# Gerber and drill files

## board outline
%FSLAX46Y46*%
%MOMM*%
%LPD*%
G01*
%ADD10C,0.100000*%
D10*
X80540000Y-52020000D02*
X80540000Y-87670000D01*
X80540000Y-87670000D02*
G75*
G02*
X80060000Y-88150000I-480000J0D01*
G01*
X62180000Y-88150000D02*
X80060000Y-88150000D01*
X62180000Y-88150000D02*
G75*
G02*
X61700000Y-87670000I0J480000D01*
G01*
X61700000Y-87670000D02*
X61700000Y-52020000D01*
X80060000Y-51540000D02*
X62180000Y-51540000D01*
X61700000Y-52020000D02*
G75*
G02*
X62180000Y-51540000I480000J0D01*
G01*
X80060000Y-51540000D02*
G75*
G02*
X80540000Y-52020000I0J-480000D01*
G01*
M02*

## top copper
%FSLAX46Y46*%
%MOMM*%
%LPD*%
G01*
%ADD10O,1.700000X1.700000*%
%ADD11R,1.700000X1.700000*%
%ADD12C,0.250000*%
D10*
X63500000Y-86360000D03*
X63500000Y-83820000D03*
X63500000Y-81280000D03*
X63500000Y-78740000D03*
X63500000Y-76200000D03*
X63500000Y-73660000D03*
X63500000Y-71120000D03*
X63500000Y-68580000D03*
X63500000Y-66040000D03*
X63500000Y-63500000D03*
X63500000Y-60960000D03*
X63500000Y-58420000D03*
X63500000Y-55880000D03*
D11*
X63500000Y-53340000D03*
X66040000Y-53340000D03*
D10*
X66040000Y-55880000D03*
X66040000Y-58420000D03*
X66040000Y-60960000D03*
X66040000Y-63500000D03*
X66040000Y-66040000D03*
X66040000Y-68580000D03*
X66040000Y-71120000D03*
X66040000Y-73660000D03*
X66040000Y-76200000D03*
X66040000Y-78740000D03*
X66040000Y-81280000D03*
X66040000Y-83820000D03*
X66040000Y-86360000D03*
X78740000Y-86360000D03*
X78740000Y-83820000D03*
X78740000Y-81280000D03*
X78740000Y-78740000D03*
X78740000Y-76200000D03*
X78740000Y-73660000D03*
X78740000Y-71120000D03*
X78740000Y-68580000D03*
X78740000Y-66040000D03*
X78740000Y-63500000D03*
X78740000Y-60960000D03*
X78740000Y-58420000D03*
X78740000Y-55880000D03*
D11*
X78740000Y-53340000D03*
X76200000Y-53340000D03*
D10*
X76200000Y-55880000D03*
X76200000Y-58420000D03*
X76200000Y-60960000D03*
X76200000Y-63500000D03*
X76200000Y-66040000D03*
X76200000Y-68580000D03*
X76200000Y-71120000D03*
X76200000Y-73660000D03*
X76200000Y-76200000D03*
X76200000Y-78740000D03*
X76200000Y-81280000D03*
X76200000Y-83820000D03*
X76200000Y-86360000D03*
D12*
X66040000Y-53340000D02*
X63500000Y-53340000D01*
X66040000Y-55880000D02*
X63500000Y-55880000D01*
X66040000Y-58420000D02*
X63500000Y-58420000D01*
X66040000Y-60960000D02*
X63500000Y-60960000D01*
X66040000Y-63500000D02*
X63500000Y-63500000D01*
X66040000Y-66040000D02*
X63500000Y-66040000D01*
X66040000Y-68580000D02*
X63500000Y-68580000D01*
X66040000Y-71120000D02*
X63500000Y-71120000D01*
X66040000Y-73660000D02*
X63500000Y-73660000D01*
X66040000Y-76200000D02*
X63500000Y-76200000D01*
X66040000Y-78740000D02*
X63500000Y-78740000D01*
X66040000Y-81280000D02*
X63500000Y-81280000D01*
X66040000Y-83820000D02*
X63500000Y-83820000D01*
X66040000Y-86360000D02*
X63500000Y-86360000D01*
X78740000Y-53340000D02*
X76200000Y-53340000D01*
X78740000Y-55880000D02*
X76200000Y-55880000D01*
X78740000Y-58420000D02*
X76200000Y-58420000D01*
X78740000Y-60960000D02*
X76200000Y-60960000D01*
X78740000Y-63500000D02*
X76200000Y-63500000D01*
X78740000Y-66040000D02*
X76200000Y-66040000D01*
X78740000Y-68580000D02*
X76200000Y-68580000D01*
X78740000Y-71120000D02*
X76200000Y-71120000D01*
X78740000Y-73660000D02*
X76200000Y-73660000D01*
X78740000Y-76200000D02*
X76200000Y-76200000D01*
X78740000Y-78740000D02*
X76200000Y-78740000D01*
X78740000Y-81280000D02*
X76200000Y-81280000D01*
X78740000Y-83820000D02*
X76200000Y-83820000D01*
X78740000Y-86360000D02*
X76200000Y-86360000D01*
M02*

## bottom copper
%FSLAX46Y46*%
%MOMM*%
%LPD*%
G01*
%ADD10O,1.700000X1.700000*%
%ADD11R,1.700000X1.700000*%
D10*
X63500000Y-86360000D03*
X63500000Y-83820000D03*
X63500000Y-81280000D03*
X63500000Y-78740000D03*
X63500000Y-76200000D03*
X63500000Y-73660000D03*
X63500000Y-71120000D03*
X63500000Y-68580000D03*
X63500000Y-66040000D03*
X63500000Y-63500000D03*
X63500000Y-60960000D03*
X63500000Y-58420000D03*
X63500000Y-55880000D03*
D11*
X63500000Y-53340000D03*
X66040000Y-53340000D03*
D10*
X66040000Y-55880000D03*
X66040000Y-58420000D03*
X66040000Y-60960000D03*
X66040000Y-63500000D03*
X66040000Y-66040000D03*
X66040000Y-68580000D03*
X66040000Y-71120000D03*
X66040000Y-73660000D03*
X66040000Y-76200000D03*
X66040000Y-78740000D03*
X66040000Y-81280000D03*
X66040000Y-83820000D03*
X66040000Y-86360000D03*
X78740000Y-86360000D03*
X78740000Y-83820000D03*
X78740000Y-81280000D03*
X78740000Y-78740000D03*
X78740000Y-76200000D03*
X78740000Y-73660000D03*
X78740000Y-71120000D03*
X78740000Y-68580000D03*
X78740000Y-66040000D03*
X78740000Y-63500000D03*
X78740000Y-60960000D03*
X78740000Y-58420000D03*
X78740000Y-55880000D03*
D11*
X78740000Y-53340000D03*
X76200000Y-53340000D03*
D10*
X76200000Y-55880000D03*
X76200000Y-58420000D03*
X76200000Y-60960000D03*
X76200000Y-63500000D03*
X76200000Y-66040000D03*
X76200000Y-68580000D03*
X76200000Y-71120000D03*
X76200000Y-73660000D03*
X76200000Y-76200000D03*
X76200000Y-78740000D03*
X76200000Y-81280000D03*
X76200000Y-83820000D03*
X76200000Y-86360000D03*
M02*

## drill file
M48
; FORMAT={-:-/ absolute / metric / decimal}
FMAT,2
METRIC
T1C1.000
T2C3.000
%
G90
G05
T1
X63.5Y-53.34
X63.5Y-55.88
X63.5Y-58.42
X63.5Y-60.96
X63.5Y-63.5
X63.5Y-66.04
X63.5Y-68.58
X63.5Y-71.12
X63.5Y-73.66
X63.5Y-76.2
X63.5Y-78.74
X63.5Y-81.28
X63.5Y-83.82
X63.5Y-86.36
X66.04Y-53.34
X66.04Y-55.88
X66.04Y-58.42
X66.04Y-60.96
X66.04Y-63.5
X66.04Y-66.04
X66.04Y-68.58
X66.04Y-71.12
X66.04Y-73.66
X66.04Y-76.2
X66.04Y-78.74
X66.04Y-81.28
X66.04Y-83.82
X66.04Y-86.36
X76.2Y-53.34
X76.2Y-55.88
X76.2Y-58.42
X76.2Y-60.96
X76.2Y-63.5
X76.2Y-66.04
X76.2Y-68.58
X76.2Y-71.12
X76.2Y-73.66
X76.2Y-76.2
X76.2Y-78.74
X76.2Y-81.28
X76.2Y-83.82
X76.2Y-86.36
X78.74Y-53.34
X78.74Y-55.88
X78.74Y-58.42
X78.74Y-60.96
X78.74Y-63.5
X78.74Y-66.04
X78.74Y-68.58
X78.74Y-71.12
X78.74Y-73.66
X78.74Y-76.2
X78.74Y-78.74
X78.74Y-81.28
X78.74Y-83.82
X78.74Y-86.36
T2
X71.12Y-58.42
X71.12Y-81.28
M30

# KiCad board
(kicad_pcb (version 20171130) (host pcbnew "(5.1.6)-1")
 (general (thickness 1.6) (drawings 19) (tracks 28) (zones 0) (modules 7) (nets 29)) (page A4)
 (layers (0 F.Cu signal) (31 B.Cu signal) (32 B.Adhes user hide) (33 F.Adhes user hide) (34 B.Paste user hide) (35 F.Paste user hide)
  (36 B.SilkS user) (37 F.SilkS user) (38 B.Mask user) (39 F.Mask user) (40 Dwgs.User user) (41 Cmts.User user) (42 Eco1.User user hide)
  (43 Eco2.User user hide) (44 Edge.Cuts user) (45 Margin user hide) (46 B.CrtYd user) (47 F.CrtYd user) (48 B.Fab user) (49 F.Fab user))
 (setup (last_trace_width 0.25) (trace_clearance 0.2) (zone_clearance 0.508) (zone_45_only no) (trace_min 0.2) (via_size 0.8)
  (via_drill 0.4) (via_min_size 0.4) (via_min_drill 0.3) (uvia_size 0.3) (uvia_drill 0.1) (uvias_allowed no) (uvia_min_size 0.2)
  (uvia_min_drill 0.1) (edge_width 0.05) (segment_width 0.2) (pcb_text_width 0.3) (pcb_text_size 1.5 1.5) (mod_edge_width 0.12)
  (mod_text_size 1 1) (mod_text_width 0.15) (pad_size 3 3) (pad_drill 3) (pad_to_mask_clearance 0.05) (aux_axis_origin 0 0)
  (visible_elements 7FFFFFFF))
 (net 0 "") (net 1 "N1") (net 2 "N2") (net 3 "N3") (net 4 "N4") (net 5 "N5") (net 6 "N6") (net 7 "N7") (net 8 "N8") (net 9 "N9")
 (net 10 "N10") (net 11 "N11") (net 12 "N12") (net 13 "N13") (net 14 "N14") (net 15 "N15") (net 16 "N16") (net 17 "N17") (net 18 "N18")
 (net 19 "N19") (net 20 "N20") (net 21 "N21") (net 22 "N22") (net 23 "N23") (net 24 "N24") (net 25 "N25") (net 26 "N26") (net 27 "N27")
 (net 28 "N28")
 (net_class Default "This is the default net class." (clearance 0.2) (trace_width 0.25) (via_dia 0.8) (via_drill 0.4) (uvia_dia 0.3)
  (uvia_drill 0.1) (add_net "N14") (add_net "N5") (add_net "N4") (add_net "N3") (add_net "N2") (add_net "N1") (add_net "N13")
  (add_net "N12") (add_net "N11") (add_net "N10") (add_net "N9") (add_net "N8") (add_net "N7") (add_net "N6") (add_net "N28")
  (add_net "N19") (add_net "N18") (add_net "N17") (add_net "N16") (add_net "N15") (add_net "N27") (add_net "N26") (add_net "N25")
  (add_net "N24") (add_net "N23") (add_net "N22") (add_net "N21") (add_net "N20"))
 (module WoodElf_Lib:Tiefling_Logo (layer F.Cu) (at 71.12 66.04 270)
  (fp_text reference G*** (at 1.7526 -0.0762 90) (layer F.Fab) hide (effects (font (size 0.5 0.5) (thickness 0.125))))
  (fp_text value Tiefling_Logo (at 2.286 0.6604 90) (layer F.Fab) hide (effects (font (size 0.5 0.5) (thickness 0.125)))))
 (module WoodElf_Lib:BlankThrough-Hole (layer F.Cu) (at 71.12 81.28)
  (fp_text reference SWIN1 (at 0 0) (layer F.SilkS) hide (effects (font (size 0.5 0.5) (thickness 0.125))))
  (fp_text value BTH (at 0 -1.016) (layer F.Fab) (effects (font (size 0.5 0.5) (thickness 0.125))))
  (pad "" np_thru_hole circle (at 0 0) (size 3 3) (drill 3) (layers *.Cu *.Mask) (solder_mask_margin 0.1) (clearance 0.1)))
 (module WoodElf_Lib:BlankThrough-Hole (layer F.Cu) (at 71.12 58.42)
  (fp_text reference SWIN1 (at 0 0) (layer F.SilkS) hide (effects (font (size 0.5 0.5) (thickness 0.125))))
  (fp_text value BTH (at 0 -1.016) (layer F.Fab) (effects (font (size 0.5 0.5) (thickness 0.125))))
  (pad "" np_thru_hole circle (at 0 0) (size 3 3) (drill 3) (layers *.Cu *.Mask) (solder_mask_margin 0.1) (clearance 0.1)))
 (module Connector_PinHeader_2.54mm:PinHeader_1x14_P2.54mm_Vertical (layer B.Cu) (at 63.5 53.34 180)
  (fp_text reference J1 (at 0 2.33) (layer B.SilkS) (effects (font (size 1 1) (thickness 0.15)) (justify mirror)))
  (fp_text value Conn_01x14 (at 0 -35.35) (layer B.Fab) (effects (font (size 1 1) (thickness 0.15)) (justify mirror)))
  (pad 14 thru_hole oval (at 0 -33.02 180) (size 1.7 1.7) (drill 1) (layers *.Cu *.Mask) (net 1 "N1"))
  (pad 13 thru_hole oval (at 0 -30.48 180) (size 1.7 1.7) (drill 1) (layers *.Cu *.Mask) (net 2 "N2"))
  (pad 12 thru_hole oval (at 0 -27.94 180) (size 1.7 1.7) (drill 1) (layers *.Cu *.Mask) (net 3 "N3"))
  (pad 11 thru_hole oval (at 0 -25.4 180) (size 1.7 1.7) (drill 1) (layers *.Cu *.Mask) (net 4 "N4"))
  (pad 10 thru_hole oval (at 0 -22.86 180) (size 1.7 1.7) (drill 1) (layers *.Cu *.Mask) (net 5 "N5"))
  (pad 9 thru_hole oval (at 0 -20.32 180) (size 1.7 1.7) (drill 1) (layers *.Cu *.Mask) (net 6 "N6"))
  (pad 8 thru_hole oval (at 0 -17.78 180) (size 1.7 1.7) (drill 1) (layers *.Cu *.Mask) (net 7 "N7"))
  (pad 7 thru_hole oval (at 0 -15.24 180) (size 1.7 1.7) (drill 1) (layers *.Cu *.Mask) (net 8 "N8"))
  (pad 6 thru_hole oval (at 0 -12.7 180) (size 1.7 1.7) (drill 1) (layers *.Cu *.Mask) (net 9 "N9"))
  (pad 5 thru_hole oval (at 0 -10.16 180) (size 1.7 1.7) (drill 1) (layers *.Cu *.Mask) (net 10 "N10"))
  (pad 4 thru_hole oval (at 0 -7.62 180) (size 1.7 1.7) (drill 1) (layers *.Cu *.Mask) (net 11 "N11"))
  (pad 3 thru_hole oval (at 0 -5.08 180) (size 1.7 1.7) (drill 1) (layers *.Cu *.Mask) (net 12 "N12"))
  (pad 2 thru_hole oval (at 0 -2.54 180) (size 1.7 1.7) (drill 1) (layers *.Cu *.Mask) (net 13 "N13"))
  (pad 1 thru_hole rect (at 0 0 180) (size 1.7 1.7) (drill 1) (layers *.Cu *.Mask) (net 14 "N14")))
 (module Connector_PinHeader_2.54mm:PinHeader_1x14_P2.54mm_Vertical (layer F.Cu) (at 66.04 53.34)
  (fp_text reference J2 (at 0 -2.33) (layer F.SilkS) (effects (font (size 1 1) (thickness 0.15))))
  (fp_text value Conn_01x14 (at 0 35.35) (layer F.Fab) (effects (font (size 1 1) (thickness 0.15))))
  (pad 1 thru_hole rect (at 0 0) (size 1.7 1.7) (drill 1) (layers *.Cu *.Mask) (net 14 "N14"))
  (pad 2 thru_hole oval (at 0 2.54) (size 1.7 1.7) (drill 1) (layers *.Cu *.Mask) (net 13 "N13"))
  (pad 3 thru_hole oval (at 0 5.08) (size 1.7 1.7) (drill 1) (layers *.Cu *.Mask) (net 12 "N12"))
  (pad 4 thru_hole oval (at 0 7.62) (size 1.7 1.7) (drill 1) (layers *.Cu *.Mask) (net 11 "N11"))
  (pad 5 thru_hole oval (at 0 10.16) (size 1.7 1.7) (drill 1) (layers *.Cu *.Mask) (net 10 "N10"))
  (pad 6 thru_hole oval (at 0 12.7) (size 1.7 1.7) (drill 1) (layers *.Cu *.Mask) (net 9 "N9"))
  (pad 7 thru_hole oval (at 0 15.24) (size 1.7 1.7) (drill 1) (layers *.Cu *.Mask) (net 8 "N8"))
  (pad 8 thru_hole oval (at 0 17.78) (size 1.7 1.7) (drill 1) (layers *.Cu *.Mask) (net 7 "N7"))
  (pad 9 thru_hole oval (at 0 20.32) (size 1.7 1.7) (drill 1) (layers *.Cu *.Mask) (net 6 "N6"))
  (pad 10 thru_hole oval (at 0 22.86) (size 1.7 1.7) (drill 1) (layers *.Cu *.Mask) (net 5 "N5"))
  (pad 11 thru_hole oval (at 0 25.4) (size 1.7 1.7) (drill 1) (layers *.Cu *.Mask) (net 4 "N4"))
  (pad 12 thru_hole oval (at 0 27.94) (size 1.7 1.7) (drill 1) (layers *.Cu *.Mask) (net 3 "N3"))
  (pad 13 thru_hole oval (at 0 30.48) (size 1.7 1.7) (drill 1) (layers *.Cu *.Mask) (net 2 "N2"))
  (pad 14 thru_hole oval (at 0 33.02) (size 1.7 1.7) (drill 1) (layers *.Cu *.Mask) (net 1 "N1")))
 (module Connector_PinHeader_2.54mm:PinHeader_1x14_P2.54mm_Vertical (layer B.Cu) (at 78.74 53.34 180)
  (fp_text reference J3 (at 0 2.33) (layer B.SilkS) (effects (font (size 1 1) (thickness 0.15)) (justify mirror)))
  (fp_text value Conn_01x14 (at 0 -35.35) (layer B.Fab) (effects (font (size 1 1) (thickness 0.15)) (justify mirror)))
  (pad 14 thru_hole oval (at 0 -33.02 180) (size 1.7 1.7) (drill 1) (layers *.Cu *.Mask) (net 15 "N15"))
  (pad 13 thru_hole oval (at 0 -30.48 180) (size 1.7 1.7) (drill 1) (layers *.Cu *.Mask) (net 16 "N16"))
  (pad 12 thru_hole oval (at 0 -27.94 180) (size 1.7 1.7) (drill 1) (layers *.Cu *.Mask) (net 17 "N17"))
  (pad 11 thru_hole oval (at 0 -25.4 180) (size 1.7 1.7) (drill 1) (layers *.Cu *.Mask) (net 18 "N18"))
  (pad 10 thru_hole oval (at 0 -22.86 180) (size 1.7 1.7) (drill 1) (layers *.Cu *.Mask) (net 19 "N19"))
  (pad 9 thru_hole oval (at 0 -20.32 180) (size 1.7 1.7) (drill 1) (layers *.Cu *.Mask) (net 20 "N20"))
  (pad 8 thru_hole oval (at 0 -17.78 180) (size 1.7 1.7) (drill 1) (layers *.Cu *.Mask) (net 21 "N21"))
  (pad 7 thru_hole oval (at 0 -15.24 180) (size 1.7 1.7) (drill 1) (layers *.Cu *.Mask) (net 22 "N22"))
  (pad 6 thru_hole oval (at 0 -12.7 180) (size 1.7 1.7) (drill 1) (layers *.Cu *.Mask) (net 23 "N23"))
  (pad 5 thru_hole oval (at 0 -10.16 180) (size 1.7 1.7) (drill 1) (layers *.Cu *.Mask) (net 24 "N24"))
  (pad 4 thru_hole oval (at 0 -7.62 180) (size 1.7 1.7) (drill 1) (layers *.Cu *.Mask) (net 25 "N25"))
  (pad 3 thru_hole oval (at 0 -5.08 180) (size 1.7 1.7) (drill 1) (layers *.Cu *.Mask) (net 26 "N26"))
  (pad 2 thru_hole oval (at 0 -2.54 180) (size 1.7 1.7) (drill 1) (layers *.Cu *.Mask) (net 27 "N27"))
  (pad 1 thru_hole rect (at 0 0 180) (size 1.7 1.7) (drill 1) (layers *.Cu *.Mask) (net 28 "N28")))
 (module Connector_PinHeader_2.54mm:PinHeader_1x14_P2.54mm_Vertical (layer F.Cu) (at 76.2 53.34)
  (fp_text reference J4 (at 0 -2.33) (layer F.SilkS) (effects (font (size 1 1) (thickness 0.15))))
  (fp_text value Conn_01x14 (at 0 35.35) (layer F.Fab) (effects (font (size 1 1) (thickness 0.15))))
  (pad 1 thru_hole rect (at 0 0) (size 1.7 1.7) (drill 1) (layers *.Cu *.Mask) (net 28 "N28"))
  (pad 2 thru_hole oval (at 0 2.54) (size 1.7 1.7) (drill 1) (layers *.Cu *.Mask) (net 27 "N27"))
  (pad 3 thru_hole oval (at 0 5.08) (size 1.7 1.7) (drill 1) (layers *.Cu *.Mask) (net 26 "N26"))
  (pad 4 thru_hole oval (at 0 7.62) (size 1.7 1.7) (drill 1) (layers *.Cu *.Mask) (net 25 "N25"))
  (pad 5 thru_hole oval (at 0 10.16) (size 1.7 1.7) (drill 1) (layers *.Cu *.Mask) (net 24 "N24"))
  (pad 6 thru_hole oval (at 0 12.7) (size 1.7 1.7) (drill 1) (layers *.Cu *.Mask) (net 23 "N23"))
  (pad 7 thru_hole oval (at 0 15.24) (size 1.7 1.7) (drill 1) (layers *.Cu *.Mask) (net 22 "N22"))
  (pad 8 thru_hole oval (at 0 17.78) (size 1.7 1.7) (drill 1) (layers *.Cu *.Mask) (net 21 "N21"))
  (pad 9 thru_hole oval (at 0 20.32) (size 1.7 1.7) (drill 1) (layers *.Cu *.Mask) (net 20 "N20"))
  (pad 10 thru_hole oval (at 0 22.86) (size 1.7 1.7) (drill 1) (layers *.Cu *.Mask) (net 19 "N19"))
  (pad 11 thru_hole oval (at 0 25.4) (size 1.7 1.7) (drill 1) (layers *.Cu *.Mask) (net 18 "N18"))
  (pad 12 thru_hole oval (at 0 27.94) (size 1.7 1.7) (drill 1) (layers *.Cu *.Mask) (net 17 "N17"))
  (pad 13 thru_hole oval (at 0 30.48) (size 1.7 1.7) (drill 1) (layers *.Cu *.Mask) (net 16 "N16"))
  (pad 14 thru_hole oval (at 0 33.02) (size 1.7 1.7) (drill 1) (layers *.Cu *.Mask) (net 15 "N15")))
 (gr_line (start 80.54 52.02) (end 80.54 87.67) (layer Edge.Cuts) (width 0.1))
 (gr_arc (start 80.06 87.67) (end 80.06 88.15) (angle -90) (layer Edge.Cuts) (width 0.1))
 (gr_line (start 62.18 88.15) (end 80.06 88.15) (layer Edge.Cuts) (width 0.1))
 (gr_arc (start 62.18 87.67) (end 61.7 87.67) (angle -90) (layer Edge.Cuts) (width 0.1))
 (gr_line (start 61.7 87.67) (end 61.7 52.02) (layer Edge.Cuts) (width 0.1))
 (gr_line (start 80.06 51.54) (end 62.18 51.54) (layer Edge.Cuts) (width 0.1))
 (gr_arc (start 62.18 52.02) (end 62.18 51.54) (angle -90) (layer Edge.Cuts) (width 0.1))
 (gr_arc (start 80.06 52.02) (end 80.54 52.02) (angle -90) (layer Edge.Cuts) (width 0.1))
 (segment (start 66.04 53.34) (end 63.5 53.34) (width 0.25) (layer F.Cu) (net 14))
 (segment (start 66.04 55.88) (end 63.5 55.88) (width 0.25) (layer F.Cu) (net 13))
 (segment (start 66.04 58.42) (end 63.5 58.42) (width 0.25) (layer F.Cu) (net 12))
 (segment (start 66.04 60.96) (end 63.5 60.96) (width 0.25) (layer F.Cu) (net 11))
 (segment (start 66.04 63.5) (end 63.5 63.5) (width 0.25) (layer F.Cu) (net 10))
 (segment (start 66.04 66.04) (end 63.5 66.04) (width 0.25) (layer F.Cu) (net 9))
 (segment (start 66.04 68.58) (end 63.5 68.58) (width 0.25) (layer F.Cu) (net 8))
 (segment (start 66.04 71.12) (end 63.5 71.12) (width 0.25) (layer F.Cu) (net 7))
 (segment (start 66.04 73.66) (end 63.5 73.66) (width 0.25) (layer F.Cu) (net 6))
 (segment (start 66.04 76.2) (end 63.5 76.2) (width 0.25) (layer F.Cu) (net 5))
 (segment (start 66.04 78.74) (end 63.5 78.74) (width 0.25) (layer F.Cu) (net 4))
 (segment (start 66.04 81.28) (end 63.5 81.28) (width 0.25) (layer F.Cu) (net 3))
 (segment (start 66.04 83.82) (end 63.5 83.82) (width 0.25) (layer F.Cu) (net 2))
 (segment (start 66.04 86.36) (end 63.5 86.36) (width 0.25) (layer F.Cu) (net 1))
 (segment (start 78.74 53.34) (end 76.2 53.34) (width 0.25) (layer F.Cu) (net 28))
 (segment (start 78.74 55.88) (end 76.2 55.88) (width 0.25) (layer F.Cu) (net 27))
 (segment (start 78.74 58.42) (end 76.2 58.42) (width 0.25) (layer F.Cu) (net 26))
 (segment (start 78.74 60.96) (end 76.2 60.96) (width 0.25) (layer F.Cu) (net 25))
 (segment (start 78.74 63.5) (end 76.2 63.5) (width 0.25) (layer F.Cu) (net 24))
 (segment (start 78.74 66.04) (end 76.2 66.04) (width 0.25) (layer F.Cu) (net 23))
 (segment (start 78.74 68.58) (end 76.2 68.58) (width 0.25) (layer F.Cu) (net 22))
 (segment (start 78.74 71.12) (end 76.2 71.12) (width 0.25) (layer F.Cu) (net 21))
 (segment (start 78.74 73.66) (end 76.2 73.66) (width 0.25) (layer F.Cu) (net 20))
 (segment (start 78.74 76.2) (end 76.2 76.2) (width 0.25) (layer F.Cu) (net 19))
 (segment (start 78.74 78.74) (end 76.2 78.74) (width 0.25) (layer F.Cu) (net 18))
 (segment (start 78.74 81.28) (end 76.2 81.28) (width 0.25) (layer F.Cu) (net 17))
 (segment (start 78.74 83.82) (end 76.2 83.82) (width 0.25) (layer F.Cu) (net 16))
 (segment (start 78.74 86.36) (end 76.2 86.36) (width 0.25) (layer F.Cu) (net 15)))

